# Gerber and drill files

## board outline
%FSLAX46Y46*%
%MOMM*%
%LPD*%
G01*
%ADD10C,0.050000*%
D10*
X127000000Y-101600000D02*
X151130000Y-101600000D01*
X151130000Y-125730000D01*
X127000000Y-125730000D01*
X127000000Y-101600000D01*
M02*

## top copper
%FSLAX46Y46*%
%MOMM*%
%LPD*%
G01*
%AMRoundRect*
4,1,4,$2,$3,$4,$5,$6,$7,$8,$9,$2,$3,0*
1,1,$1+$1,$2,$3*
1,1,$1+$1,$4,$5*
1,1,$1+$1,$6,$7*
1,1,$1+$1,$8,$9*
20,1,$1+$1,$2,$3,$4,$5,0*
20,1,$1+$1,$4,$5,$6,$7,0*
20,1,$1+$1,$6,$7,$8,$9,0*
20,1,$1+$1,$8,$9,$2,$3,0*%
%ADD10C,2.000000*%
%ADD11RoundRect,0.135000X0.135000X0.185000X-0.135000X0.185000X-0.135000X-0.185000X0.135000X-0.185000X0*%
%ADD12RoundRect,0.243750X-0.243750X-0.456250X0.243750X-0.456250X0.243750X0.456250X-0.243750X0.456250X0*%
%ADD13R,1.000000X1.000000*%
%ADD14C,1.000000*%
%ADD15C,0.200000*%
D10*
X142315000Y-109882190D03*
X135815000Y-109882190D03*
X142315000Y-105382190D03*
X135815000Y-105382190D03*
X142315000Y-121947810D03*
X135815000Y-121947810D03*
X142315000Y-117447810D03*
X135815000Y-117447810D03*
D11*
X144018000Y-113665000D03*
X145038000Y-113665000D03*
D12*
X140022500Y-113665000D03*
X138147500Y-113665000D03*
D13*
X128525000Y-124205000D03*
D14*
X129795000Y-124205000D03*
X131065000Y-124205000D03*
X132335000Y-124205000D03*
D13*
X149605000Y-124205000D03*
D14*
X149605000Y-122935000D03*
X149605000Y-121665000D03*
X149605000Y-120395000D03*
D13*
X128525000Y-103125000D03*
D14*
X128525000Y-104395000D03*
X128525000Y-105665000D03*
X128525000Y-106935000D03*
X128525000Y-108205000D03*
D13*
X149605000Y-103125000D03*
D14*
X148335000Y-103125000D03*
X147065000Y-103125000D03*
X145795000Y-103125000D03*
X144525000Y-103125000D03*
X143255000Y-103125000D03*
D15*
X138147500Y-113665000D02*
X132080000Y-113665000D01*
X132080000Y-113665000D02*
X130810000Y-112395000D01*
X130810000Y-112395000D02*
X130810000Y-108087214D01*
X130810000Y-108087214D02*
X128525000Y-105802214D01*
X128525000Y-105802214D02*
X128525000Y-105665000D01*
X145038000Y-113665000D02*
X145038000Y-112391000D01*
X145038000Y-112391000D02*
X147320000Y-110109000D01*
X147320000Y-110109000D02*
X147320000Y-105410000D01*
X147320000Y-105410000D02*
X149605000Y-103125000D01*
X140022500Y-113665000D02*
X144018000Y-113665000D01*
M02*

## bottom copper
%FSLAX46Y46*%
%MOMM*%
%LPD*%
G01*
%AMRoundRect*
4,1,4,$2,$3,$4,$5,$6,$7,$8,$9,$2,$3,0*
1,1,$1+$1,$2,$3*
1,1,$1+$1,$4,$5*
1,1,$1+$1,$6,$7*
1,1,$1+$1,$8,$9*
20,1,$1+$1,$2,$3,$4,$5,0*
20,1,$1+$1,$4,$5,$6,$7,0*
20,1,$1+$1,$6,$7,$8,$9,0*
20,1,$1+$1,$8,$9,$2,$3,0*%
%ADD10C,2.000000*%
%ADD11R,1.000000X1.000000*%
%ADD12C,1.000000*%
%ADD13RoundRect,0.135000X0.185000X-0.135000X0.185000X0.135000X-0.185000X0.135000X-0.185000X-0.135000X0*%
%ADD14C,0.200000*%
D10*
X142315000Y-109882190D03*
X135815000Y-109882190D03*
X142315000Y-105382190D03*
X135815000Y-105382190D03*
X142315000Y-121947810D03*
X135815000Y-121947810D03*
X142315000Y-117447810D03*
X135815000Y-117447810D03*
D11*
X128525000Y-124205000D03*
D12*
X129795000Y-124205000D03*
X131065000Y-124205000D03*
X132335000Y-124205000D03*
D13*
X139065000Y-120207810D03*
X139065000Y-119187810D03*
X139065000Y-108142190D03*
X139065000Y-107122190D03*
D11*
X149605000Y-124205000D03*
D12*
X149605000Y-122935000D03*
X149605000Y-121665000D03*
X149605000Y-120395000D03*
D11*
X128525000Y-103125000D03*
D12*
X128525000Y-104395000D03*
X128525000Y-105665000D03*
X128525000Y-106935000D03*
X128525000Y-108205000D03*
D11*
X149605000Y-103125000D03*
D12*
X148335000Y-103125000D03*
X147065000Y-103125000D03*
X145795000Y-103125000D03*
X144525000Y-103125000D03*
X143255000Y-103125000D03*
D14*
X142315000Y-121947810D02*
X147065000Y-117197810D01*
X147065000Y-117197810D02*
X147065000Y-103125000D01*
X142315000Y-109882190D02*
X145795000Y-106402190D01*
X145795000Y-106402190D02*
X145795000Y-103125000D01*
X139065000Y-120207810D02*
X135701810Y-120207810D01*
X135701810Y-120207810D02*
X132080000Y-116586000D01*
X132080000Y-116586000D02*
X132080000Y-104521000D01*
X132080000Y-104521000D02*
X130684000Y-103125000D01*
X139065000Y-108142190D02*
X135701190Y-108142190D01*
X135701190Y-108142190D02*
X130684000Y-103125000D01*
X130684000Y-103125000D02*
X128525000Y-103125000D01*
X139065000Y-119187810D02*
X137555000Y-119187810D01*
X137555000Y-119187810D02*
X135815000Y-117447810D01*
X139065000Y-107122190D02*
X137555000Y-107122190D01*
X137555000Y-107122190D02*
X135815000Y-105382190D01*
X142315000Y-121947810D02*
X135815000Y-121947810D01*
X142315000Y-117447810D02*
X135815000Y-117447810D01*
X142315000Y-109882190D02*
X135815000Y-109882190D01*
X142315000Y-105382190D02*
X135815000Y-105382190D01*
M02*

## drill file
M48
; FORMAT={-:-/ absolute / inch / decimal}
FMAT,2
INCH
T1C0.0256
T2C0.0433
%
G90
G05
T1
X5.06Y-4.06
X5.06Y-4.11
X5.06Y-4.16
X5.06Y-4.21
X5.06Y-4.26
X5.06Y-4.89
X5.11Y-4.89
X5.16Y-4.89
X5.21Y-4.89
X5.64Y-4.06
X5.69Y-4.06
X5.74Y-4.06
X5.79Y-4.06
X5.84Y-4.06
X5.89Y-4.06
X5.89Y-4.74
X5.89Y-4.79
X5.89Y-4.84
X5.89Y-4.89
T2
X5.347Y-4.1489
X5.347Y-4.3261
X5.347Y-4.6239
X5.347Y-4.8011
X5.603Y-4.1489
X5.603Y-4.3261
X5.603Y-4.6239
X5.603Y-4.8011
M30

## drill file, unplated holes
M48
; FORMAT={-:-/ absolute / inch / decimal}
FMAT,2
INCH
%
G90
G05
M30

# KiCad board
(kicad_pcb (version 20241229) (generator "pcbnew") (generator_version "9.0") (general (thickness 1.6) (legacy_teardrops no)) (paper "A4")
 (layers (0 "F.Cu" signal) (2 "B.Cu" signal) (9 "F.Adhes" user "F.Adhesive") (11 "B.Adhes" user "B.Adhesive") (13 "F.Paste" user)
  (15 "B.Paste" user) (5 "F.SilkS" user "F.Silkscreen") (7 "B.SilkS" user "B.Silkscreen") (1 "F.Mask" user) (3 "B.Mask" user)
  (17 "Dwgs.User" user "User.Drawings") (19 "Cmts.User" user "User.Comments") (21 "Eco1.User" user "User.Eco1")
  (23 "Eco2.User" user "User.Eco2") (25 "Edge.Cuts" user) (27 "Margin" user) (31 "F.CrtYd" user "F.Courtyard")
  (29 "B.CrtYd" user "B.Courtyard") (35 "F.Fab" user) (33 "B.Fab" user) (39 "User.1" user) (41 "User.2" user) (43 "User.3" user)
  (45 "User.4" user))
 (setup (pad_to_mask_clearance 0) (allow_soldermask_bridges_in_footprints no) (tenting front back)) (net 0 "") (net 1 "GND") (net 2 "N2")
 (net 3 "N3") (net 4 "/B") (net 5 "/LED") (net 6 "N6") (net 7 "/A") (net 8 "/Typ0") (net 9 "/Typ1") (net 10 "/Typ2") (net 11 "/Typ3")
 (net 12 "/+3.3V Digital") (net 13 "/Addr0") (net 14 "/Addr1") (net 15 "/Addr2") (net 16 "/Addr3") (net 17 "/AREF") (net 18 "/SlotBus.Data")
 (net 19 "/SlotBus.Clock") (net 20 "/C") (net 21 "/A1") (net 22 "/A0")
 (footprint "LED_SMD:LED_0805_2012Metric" (layer "F.Cu") (at 139.085 113.665)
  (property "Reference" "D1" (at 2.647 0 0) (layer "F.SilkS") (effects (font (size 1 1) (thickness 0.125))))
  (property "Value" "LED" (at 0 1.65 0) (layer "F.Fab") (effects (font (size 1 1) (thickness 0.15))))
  (pad "1" smd roundrect (at -0.9375 0) (size 0.975 1.4) (layers "F.Cu" "F.Mask" "F.Paste") (roundrect_rratio 0.25) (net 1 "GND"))
  (pad "2" smd roundrect (at 0.9375 0) (size 0.975 1.4) (layers "F.Cu" "F.Mask" "F.Paste") (roundrect_rratio 0.25) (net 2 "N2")))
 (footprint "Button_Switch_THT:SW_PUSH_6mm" (layer "F.Cu") (at 135.815 117.44781)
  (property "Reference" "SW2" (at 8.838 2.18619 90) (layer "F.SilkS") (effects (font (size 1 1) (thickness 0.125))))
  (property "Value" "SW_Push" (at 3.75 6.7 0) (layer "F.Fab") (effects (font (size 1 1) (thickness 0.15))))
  (pad "1" thru_hole circle (at 0 0 90) (size 2 2) (drill 1.1) (layers "*.Cu" "*.Mask") (remove_unused_layers no) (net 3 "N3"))
  (pad "1" thru_hole circle (at 6.5 0 90) (size 2 2) (drill 1.1) (layers "*.Cu" "*.Mask") (remove_unused_layers no) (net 3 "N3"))
  (pad "2" thru_hole circle (at 0 4.5 90) (size 2 2) (drill 1.1) (layers "*.Cu" "*.Mask") (remove_unused_layers no) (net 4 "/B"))
  (pad "2" thru_hole circle (at 6.5 4.5 90) (size 2 2) (drill 1.1) (layers "*.Cu" "*.Mask") (remove_unused_layers no) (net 4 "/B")))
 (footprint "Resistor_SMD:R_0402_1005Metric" (layer "F.Cu") (at 144.528 113.665 180)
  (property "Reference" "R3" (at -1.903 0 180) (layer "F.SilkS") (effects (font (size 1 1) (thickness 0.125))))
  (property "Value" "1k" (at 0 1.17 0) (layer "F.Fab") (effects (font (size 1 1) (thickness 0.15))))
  (pad "1" smd roundrect (at -0.51 0 180) (size 0.54 0.64) (layers "F.Cu" "F.Mask" "F.Paste") (roundrect_rratio 0.25) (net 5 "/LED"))
  (pad "2" smd roundrect (at 0.51 0 180) (size 0.54 0.64) (layers "F.Cu" "F.Mask" "F.Paste") (roundrect_rratio 0.25) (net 2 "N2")))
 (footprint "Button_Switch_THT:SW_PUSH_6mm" (layer "F.Cu") (at 135.815 105.38219)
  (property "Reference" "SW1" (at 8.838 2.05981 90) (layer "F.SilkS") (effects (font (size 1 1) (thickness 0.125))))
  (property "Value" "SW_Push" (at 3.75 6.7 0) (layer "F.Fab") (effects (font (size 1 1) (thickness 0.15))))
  (pad "1" thru_hole circle (at 0 0 90) (size 2 2) (drill 1.1) (layers "*.Cu" "*.Mask") (remove_unused_layers no) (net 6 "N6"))
  (pad "1" thru_hole circle (at 6.5 0 90) (size 2 2) (drill 1.1) (layers "*.Cu" "*.Mask") (remove_unused_layers no) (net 6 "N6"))
  (pad "2" thru_hole circle (at 0 4.5 90) (size 2 2) (drill 1.1) (layers "*.Cu" "*.Mask") (remove_unused_layers no) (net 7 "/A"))
  (pad "2" thru_hole circle (at 6.5 4.5 90) (size 2 2) (drill 1.1) (layers "*.Cu" "*.Mask") (remove_unused_layers no) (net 7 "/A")))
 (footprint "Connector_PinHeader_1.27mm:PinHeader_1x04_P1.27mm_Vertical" (layer "B.Cu") (at 128.525 124.205 -90)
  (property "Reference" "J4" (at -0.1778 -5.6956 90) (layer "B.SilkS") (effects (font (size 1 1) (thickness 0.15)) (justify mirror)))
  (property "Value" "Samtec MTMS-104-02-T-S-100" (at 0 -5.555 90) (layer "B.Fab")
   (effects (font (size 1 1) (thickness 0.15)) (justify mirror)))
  (pad "1" thru_hole rect (at 0 0 270) (size 1 1) (drill 0.65) (layers "*.Cu" "*.Mask") (remove_unused_layers no) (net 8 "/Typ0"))
  (pad "2" thru_hole circle (at 0 -1.27 270) (size 1 1) (drill 0.65) (layers "*.Cu" "*.Mask") (remove_unused_layers no) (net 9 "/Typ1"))
  (pad "3" thru_hole circle (at 0 -2.54 270) (size 1 1) (drill 0.65) (layers "*.Cu" "*.Mask") (remove_unused_layers no) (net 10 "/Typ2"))
  (pad "4" thru_hole circle (at 0 -3.81 270) (size 1 1) (drill 0.65) (layers "*.Cu" "*.Mask") (remove_unused_layers no) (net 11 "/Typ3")))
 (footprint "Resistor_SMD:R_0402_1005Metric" (layer "B.Cu") (at 139.065 119.69781 90)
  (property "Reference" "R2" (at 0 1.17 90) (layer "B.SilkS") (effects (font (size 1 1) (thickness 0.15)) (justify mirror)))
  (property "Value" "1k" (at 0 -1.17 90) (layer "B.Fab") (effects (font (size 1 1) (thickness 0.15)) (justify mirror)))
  (pad "1" smd roundrect (at -0.51 0 90) (size 0.54 0.64) (layers "B.Cu" "B.Mask" "B.Paste") (roundrect_rratio 0.25)
   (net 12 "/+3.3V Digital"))
  (pad "2" smd roundrect (at 0.51 0 90) (size 0.54 0.64) (layers "B.Cu" "B.Mask" "B.Paste") (roundrect_rratio 0.25) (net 3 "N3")))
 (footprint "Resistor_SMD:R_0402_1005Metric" (layer "B.Cu") (at 139.065 107.63219 90)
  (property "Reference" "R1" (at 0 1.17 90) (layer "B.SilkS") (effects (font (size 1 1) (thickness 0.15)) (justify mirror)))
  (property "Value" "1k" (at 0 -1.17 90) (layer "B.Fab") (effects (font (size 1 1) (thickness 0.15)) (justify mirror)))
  (pad "1" smd roundrect (at -0.51 0 90) (size 0.54 0.64) (layers "B.Cu" "B.Mask" "B.Paste") (roundrect_rratio 0.25)
   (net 12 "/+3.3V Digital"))
  (pad "2" smd roundrect (at 0.51 0 90) (size 0.54 0.64) (layers "B.Cu" "B.Mask" "B.Paste") (roundrect_rratio 0.25) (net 6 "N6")))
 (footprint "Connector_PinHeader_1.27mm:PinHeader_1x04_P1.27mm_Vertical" (layer "B.Cu") (at 149.605 124.205)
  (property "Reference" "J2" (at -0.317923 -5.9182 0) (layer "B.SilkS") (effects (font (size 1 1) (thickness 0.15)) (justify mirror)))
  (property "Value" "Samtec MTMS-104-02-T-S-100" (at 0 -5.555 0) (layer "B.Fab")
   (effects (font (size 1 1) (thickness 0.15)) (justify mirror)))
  (pad "1" thru_hole rect (at 0 0) (size 1 1) (drill 0.65) (layers "*.Cu" "*.Mask") (remove_unused_layers no) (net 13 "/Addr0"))
  (pad "2" thru_hole circle (at 0 -1.27) (size 1 1) (drill 0.65) (layers "*.Cu" "*.Mask") (remove_unused_layers no) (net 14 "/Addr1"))
  (pad "3" thru_hole circle (at 0 -2.54) (size 1 1) (drill 0.65) (layers "*.Cu" "*.Mask") (remove_unused_layers no) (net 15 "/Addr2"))
  (pad "4" thru_hole circle (at 0 -3.81) (size 1 1) (drill 0.65) (layers "*.Cu" "*.Mask") (remove_unused_layers no) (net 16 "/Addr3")))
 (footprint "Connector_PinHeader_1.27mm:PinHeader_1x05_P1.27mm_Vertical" (layer "B.Cu") (at 128.525 103.125 180)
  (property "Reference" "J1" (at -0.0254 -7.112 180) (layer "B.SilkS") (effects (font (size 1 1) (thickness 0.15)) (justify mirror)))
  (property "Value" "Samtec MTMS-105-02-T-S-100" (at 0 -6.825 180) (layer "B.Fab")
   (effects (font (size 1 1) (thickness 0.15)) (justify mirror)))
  (pad "1" thru_hole rect (at 0 0 180) (size 1 1) (drill 0.65) (layers "*.Cu" "*.Mask") (remove_unused_layers no) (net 12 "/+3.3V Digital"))
  (pad "2" thru_hole circle (at 0 -1.27 180) (size 1 1) (drill 0.65) (layers "*.Cu" "*.Mask") (remove_unused_layers no) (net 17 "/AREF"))
  (pad "3" thru_hole circle (at 0 -2.54 180) (size 1 1) (drill 0.65) (layers "*.Cu" "*.Mask") (remove_unused_layers no) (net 1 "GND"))
  (pad "4" thru_hole circle (at 0 -3.81 180) (size 1 1) (drill 0.65) (layers "*.Cu" "*.Mask") (remove_unused_layers no)
   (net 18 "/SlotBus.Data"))
  (pad "5" thru_hole circle (at 0 -5.08 180) (size 1 1) (drill 0.65) (layers "*.Cu" "*.Mask") (remove_unused_layers no)
   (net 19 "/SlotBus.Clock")))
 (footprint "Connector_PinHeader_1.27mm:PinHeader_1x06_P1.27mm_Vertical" (layer "B.Cu") (at 149.605 103.125 90)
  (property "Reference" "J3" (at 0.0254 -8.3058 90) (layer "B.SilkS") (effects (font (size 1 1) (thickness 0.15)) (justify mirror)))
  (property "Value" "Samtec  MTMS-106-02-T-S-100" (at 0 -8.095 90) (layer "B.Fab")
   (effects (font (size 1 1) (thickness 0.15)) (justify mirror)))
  (pad "1" thru_hole rect (at 0 0 90) (size 1 1) (drill 0.65) (layers "*.Cu" "*.Mask") (remove_unused_layers no) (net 5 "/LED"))
  (pad "2" thru_hole circle (at 0 -1.27 90) (size 1 1) (drill 0.65) (layers "*.Cu" "*.Mask") (remove_unused_layers no) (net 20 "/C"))
  (pad "3" thru_hole circle (at 0 -2.54 90) (size 1 1) (drill 0.65) (layers "*.Cu" "*.Mask") (remove_unused_layers no) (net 4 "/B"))
  (pad "4" thru_hole circle (at 0 -3.81 90) (size 1 1) (drill 0.65) (layers "*.Cu" "*.Mask") (remove_unused_layers no) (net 7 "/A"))
  (pad "5" thru_hole circle (at 0 -5.08 90) (size 1 1) (drill 0.65) (layers "*.Cu" "*.Mask") (remove_unused_layers no) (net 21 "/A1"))
  (pad "6" thru_hole circle (at 0 -6.35 90) (size 1 1) (drill 0.65) (layers "*.Cu" "*.Mask") (remove_unused_layers no) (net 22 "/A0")))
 (gr_rect (start 127 101.6) (end 151.13 125.73) (stroke (width 0.05) (type solid)) (fill no) (layer "Edge.Cuts"))
 (segment (start 132.08 113.665) (end 130.81 112.395) (width 0.2) (layer "F.Cu") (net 1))
 (segment (start 128.525 105.802214) (end 128.525 105.665) (width 0.2) (layer "F.Cu") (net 1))
 (segment (start 130.81 108.087214) (end 128.525 105.802214) (width 0.2) (layer "F.Cu") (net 1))
 (segment (start 138.1475 113.665) (end 132.08 113.665) (width 0.2) (layer "F.Cu") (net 1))
 (segment (start 130.81 112.395) (end 130.81 108.087214) (width 0.2) (layer "F.Cu") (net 1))
 (segment (start 140.0225 113.665) (end 144.018 113.665) (width 0.2) (layer "F.Cu") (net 2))
 (segment (start 130.684 103.125) (end 128.525 103.125) (width 0.2) (layer "B.Cu") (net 12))
 (segment (start 135.70181 120.20781) (end 132.08 116.586) (width 0.2) (layer "B.Cu") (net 12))
 (segment (start 139.065 120.20781) (end 135.70181 120.20781) (width 0.2) (layer "B.Cu") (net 12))
 (segment (start 132.08 116.586) (end 132.08 104.521) (width 0.2) (layer "B.Cu") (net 12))
 (segment (start 132.08 104.521) (end 130.684 103.125) (width 0.2) (layer "B.Cu") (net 12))
 (segment (start 135.70119 108.14219) (end 130.684 103.125) (width 0.2) (layer "B.Cu") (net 12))
 (segment (start 139.065 108.14219) (end 135.70119 108.14219) (width 0.2) (layer "B.Cu") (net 12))
 (segment (start 142.315 121.94781) (end 135.815 121.94781) (width 0.2) (layer "B.Cu") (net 4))
 (segment (start 142.315 121.94781) (end 147.065 117.19781) (width 0.2) (layer "B.Cu") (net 4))
 (segment (start 147.065 117.19781) (end 147.065 103.125) (width 0.2) (layer "B.Cu") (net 4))
 (segment (start 147.32 105.41) (end 149.605 103.125) (width 0.2) (layer "F.Cu") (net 5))
 (segment (start 145.038 113.665) (end 145.038 112.391) (width 0.2) (layer "F.Cu") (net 5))
 (segment (start 147.32 110.109) (end 147.32 105.41) (width 0.2) (layer "F.Cu") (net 5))
 (segment (start 145.038 112.391) (end 147.32 110.109) (width 0.2) (layer "F.Cu") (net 5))
 (segment (start 142.315 109.88219) (end 135.815 109.88219) (width 0.2) (layer "B.Cu") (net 7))
 (segment (start 145.795 106.40219) (end 145.795 103.125) (width 0.2) (layer "B.Cu") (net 7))
 (segment (start 142.315 109.88219) (end 145.795 106.40219) (width 0.2) (layer "B.Cu") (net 7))
 (segment (start 137.555 107.12219) (end 135.815 105.38219) (width 0.2) (layer "B.Cu") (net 6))
 (segment (start 142.315 105.38219) (end 135.815 105.38219) (width 0.2) (layer "B.Cu") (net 6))
 (segment (start 139.065 107.12219) (end 137.555 107.12219) (width 0.2) (layer "B.Cu") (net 6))
 (segment (start 139.065 119.18781) (end 137.555 119.18781) (width 0.2) (layer "B.Cu") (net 3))
 (segment (start 142.315 117.44781) (end 135.815 117.44781) (width 0.2) (layer "B.Cu") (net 3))
 (segment (start 137.555 119.18781) (end 135.815 117.44781) (width 0.2) (layer "B.Cu") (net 3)))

